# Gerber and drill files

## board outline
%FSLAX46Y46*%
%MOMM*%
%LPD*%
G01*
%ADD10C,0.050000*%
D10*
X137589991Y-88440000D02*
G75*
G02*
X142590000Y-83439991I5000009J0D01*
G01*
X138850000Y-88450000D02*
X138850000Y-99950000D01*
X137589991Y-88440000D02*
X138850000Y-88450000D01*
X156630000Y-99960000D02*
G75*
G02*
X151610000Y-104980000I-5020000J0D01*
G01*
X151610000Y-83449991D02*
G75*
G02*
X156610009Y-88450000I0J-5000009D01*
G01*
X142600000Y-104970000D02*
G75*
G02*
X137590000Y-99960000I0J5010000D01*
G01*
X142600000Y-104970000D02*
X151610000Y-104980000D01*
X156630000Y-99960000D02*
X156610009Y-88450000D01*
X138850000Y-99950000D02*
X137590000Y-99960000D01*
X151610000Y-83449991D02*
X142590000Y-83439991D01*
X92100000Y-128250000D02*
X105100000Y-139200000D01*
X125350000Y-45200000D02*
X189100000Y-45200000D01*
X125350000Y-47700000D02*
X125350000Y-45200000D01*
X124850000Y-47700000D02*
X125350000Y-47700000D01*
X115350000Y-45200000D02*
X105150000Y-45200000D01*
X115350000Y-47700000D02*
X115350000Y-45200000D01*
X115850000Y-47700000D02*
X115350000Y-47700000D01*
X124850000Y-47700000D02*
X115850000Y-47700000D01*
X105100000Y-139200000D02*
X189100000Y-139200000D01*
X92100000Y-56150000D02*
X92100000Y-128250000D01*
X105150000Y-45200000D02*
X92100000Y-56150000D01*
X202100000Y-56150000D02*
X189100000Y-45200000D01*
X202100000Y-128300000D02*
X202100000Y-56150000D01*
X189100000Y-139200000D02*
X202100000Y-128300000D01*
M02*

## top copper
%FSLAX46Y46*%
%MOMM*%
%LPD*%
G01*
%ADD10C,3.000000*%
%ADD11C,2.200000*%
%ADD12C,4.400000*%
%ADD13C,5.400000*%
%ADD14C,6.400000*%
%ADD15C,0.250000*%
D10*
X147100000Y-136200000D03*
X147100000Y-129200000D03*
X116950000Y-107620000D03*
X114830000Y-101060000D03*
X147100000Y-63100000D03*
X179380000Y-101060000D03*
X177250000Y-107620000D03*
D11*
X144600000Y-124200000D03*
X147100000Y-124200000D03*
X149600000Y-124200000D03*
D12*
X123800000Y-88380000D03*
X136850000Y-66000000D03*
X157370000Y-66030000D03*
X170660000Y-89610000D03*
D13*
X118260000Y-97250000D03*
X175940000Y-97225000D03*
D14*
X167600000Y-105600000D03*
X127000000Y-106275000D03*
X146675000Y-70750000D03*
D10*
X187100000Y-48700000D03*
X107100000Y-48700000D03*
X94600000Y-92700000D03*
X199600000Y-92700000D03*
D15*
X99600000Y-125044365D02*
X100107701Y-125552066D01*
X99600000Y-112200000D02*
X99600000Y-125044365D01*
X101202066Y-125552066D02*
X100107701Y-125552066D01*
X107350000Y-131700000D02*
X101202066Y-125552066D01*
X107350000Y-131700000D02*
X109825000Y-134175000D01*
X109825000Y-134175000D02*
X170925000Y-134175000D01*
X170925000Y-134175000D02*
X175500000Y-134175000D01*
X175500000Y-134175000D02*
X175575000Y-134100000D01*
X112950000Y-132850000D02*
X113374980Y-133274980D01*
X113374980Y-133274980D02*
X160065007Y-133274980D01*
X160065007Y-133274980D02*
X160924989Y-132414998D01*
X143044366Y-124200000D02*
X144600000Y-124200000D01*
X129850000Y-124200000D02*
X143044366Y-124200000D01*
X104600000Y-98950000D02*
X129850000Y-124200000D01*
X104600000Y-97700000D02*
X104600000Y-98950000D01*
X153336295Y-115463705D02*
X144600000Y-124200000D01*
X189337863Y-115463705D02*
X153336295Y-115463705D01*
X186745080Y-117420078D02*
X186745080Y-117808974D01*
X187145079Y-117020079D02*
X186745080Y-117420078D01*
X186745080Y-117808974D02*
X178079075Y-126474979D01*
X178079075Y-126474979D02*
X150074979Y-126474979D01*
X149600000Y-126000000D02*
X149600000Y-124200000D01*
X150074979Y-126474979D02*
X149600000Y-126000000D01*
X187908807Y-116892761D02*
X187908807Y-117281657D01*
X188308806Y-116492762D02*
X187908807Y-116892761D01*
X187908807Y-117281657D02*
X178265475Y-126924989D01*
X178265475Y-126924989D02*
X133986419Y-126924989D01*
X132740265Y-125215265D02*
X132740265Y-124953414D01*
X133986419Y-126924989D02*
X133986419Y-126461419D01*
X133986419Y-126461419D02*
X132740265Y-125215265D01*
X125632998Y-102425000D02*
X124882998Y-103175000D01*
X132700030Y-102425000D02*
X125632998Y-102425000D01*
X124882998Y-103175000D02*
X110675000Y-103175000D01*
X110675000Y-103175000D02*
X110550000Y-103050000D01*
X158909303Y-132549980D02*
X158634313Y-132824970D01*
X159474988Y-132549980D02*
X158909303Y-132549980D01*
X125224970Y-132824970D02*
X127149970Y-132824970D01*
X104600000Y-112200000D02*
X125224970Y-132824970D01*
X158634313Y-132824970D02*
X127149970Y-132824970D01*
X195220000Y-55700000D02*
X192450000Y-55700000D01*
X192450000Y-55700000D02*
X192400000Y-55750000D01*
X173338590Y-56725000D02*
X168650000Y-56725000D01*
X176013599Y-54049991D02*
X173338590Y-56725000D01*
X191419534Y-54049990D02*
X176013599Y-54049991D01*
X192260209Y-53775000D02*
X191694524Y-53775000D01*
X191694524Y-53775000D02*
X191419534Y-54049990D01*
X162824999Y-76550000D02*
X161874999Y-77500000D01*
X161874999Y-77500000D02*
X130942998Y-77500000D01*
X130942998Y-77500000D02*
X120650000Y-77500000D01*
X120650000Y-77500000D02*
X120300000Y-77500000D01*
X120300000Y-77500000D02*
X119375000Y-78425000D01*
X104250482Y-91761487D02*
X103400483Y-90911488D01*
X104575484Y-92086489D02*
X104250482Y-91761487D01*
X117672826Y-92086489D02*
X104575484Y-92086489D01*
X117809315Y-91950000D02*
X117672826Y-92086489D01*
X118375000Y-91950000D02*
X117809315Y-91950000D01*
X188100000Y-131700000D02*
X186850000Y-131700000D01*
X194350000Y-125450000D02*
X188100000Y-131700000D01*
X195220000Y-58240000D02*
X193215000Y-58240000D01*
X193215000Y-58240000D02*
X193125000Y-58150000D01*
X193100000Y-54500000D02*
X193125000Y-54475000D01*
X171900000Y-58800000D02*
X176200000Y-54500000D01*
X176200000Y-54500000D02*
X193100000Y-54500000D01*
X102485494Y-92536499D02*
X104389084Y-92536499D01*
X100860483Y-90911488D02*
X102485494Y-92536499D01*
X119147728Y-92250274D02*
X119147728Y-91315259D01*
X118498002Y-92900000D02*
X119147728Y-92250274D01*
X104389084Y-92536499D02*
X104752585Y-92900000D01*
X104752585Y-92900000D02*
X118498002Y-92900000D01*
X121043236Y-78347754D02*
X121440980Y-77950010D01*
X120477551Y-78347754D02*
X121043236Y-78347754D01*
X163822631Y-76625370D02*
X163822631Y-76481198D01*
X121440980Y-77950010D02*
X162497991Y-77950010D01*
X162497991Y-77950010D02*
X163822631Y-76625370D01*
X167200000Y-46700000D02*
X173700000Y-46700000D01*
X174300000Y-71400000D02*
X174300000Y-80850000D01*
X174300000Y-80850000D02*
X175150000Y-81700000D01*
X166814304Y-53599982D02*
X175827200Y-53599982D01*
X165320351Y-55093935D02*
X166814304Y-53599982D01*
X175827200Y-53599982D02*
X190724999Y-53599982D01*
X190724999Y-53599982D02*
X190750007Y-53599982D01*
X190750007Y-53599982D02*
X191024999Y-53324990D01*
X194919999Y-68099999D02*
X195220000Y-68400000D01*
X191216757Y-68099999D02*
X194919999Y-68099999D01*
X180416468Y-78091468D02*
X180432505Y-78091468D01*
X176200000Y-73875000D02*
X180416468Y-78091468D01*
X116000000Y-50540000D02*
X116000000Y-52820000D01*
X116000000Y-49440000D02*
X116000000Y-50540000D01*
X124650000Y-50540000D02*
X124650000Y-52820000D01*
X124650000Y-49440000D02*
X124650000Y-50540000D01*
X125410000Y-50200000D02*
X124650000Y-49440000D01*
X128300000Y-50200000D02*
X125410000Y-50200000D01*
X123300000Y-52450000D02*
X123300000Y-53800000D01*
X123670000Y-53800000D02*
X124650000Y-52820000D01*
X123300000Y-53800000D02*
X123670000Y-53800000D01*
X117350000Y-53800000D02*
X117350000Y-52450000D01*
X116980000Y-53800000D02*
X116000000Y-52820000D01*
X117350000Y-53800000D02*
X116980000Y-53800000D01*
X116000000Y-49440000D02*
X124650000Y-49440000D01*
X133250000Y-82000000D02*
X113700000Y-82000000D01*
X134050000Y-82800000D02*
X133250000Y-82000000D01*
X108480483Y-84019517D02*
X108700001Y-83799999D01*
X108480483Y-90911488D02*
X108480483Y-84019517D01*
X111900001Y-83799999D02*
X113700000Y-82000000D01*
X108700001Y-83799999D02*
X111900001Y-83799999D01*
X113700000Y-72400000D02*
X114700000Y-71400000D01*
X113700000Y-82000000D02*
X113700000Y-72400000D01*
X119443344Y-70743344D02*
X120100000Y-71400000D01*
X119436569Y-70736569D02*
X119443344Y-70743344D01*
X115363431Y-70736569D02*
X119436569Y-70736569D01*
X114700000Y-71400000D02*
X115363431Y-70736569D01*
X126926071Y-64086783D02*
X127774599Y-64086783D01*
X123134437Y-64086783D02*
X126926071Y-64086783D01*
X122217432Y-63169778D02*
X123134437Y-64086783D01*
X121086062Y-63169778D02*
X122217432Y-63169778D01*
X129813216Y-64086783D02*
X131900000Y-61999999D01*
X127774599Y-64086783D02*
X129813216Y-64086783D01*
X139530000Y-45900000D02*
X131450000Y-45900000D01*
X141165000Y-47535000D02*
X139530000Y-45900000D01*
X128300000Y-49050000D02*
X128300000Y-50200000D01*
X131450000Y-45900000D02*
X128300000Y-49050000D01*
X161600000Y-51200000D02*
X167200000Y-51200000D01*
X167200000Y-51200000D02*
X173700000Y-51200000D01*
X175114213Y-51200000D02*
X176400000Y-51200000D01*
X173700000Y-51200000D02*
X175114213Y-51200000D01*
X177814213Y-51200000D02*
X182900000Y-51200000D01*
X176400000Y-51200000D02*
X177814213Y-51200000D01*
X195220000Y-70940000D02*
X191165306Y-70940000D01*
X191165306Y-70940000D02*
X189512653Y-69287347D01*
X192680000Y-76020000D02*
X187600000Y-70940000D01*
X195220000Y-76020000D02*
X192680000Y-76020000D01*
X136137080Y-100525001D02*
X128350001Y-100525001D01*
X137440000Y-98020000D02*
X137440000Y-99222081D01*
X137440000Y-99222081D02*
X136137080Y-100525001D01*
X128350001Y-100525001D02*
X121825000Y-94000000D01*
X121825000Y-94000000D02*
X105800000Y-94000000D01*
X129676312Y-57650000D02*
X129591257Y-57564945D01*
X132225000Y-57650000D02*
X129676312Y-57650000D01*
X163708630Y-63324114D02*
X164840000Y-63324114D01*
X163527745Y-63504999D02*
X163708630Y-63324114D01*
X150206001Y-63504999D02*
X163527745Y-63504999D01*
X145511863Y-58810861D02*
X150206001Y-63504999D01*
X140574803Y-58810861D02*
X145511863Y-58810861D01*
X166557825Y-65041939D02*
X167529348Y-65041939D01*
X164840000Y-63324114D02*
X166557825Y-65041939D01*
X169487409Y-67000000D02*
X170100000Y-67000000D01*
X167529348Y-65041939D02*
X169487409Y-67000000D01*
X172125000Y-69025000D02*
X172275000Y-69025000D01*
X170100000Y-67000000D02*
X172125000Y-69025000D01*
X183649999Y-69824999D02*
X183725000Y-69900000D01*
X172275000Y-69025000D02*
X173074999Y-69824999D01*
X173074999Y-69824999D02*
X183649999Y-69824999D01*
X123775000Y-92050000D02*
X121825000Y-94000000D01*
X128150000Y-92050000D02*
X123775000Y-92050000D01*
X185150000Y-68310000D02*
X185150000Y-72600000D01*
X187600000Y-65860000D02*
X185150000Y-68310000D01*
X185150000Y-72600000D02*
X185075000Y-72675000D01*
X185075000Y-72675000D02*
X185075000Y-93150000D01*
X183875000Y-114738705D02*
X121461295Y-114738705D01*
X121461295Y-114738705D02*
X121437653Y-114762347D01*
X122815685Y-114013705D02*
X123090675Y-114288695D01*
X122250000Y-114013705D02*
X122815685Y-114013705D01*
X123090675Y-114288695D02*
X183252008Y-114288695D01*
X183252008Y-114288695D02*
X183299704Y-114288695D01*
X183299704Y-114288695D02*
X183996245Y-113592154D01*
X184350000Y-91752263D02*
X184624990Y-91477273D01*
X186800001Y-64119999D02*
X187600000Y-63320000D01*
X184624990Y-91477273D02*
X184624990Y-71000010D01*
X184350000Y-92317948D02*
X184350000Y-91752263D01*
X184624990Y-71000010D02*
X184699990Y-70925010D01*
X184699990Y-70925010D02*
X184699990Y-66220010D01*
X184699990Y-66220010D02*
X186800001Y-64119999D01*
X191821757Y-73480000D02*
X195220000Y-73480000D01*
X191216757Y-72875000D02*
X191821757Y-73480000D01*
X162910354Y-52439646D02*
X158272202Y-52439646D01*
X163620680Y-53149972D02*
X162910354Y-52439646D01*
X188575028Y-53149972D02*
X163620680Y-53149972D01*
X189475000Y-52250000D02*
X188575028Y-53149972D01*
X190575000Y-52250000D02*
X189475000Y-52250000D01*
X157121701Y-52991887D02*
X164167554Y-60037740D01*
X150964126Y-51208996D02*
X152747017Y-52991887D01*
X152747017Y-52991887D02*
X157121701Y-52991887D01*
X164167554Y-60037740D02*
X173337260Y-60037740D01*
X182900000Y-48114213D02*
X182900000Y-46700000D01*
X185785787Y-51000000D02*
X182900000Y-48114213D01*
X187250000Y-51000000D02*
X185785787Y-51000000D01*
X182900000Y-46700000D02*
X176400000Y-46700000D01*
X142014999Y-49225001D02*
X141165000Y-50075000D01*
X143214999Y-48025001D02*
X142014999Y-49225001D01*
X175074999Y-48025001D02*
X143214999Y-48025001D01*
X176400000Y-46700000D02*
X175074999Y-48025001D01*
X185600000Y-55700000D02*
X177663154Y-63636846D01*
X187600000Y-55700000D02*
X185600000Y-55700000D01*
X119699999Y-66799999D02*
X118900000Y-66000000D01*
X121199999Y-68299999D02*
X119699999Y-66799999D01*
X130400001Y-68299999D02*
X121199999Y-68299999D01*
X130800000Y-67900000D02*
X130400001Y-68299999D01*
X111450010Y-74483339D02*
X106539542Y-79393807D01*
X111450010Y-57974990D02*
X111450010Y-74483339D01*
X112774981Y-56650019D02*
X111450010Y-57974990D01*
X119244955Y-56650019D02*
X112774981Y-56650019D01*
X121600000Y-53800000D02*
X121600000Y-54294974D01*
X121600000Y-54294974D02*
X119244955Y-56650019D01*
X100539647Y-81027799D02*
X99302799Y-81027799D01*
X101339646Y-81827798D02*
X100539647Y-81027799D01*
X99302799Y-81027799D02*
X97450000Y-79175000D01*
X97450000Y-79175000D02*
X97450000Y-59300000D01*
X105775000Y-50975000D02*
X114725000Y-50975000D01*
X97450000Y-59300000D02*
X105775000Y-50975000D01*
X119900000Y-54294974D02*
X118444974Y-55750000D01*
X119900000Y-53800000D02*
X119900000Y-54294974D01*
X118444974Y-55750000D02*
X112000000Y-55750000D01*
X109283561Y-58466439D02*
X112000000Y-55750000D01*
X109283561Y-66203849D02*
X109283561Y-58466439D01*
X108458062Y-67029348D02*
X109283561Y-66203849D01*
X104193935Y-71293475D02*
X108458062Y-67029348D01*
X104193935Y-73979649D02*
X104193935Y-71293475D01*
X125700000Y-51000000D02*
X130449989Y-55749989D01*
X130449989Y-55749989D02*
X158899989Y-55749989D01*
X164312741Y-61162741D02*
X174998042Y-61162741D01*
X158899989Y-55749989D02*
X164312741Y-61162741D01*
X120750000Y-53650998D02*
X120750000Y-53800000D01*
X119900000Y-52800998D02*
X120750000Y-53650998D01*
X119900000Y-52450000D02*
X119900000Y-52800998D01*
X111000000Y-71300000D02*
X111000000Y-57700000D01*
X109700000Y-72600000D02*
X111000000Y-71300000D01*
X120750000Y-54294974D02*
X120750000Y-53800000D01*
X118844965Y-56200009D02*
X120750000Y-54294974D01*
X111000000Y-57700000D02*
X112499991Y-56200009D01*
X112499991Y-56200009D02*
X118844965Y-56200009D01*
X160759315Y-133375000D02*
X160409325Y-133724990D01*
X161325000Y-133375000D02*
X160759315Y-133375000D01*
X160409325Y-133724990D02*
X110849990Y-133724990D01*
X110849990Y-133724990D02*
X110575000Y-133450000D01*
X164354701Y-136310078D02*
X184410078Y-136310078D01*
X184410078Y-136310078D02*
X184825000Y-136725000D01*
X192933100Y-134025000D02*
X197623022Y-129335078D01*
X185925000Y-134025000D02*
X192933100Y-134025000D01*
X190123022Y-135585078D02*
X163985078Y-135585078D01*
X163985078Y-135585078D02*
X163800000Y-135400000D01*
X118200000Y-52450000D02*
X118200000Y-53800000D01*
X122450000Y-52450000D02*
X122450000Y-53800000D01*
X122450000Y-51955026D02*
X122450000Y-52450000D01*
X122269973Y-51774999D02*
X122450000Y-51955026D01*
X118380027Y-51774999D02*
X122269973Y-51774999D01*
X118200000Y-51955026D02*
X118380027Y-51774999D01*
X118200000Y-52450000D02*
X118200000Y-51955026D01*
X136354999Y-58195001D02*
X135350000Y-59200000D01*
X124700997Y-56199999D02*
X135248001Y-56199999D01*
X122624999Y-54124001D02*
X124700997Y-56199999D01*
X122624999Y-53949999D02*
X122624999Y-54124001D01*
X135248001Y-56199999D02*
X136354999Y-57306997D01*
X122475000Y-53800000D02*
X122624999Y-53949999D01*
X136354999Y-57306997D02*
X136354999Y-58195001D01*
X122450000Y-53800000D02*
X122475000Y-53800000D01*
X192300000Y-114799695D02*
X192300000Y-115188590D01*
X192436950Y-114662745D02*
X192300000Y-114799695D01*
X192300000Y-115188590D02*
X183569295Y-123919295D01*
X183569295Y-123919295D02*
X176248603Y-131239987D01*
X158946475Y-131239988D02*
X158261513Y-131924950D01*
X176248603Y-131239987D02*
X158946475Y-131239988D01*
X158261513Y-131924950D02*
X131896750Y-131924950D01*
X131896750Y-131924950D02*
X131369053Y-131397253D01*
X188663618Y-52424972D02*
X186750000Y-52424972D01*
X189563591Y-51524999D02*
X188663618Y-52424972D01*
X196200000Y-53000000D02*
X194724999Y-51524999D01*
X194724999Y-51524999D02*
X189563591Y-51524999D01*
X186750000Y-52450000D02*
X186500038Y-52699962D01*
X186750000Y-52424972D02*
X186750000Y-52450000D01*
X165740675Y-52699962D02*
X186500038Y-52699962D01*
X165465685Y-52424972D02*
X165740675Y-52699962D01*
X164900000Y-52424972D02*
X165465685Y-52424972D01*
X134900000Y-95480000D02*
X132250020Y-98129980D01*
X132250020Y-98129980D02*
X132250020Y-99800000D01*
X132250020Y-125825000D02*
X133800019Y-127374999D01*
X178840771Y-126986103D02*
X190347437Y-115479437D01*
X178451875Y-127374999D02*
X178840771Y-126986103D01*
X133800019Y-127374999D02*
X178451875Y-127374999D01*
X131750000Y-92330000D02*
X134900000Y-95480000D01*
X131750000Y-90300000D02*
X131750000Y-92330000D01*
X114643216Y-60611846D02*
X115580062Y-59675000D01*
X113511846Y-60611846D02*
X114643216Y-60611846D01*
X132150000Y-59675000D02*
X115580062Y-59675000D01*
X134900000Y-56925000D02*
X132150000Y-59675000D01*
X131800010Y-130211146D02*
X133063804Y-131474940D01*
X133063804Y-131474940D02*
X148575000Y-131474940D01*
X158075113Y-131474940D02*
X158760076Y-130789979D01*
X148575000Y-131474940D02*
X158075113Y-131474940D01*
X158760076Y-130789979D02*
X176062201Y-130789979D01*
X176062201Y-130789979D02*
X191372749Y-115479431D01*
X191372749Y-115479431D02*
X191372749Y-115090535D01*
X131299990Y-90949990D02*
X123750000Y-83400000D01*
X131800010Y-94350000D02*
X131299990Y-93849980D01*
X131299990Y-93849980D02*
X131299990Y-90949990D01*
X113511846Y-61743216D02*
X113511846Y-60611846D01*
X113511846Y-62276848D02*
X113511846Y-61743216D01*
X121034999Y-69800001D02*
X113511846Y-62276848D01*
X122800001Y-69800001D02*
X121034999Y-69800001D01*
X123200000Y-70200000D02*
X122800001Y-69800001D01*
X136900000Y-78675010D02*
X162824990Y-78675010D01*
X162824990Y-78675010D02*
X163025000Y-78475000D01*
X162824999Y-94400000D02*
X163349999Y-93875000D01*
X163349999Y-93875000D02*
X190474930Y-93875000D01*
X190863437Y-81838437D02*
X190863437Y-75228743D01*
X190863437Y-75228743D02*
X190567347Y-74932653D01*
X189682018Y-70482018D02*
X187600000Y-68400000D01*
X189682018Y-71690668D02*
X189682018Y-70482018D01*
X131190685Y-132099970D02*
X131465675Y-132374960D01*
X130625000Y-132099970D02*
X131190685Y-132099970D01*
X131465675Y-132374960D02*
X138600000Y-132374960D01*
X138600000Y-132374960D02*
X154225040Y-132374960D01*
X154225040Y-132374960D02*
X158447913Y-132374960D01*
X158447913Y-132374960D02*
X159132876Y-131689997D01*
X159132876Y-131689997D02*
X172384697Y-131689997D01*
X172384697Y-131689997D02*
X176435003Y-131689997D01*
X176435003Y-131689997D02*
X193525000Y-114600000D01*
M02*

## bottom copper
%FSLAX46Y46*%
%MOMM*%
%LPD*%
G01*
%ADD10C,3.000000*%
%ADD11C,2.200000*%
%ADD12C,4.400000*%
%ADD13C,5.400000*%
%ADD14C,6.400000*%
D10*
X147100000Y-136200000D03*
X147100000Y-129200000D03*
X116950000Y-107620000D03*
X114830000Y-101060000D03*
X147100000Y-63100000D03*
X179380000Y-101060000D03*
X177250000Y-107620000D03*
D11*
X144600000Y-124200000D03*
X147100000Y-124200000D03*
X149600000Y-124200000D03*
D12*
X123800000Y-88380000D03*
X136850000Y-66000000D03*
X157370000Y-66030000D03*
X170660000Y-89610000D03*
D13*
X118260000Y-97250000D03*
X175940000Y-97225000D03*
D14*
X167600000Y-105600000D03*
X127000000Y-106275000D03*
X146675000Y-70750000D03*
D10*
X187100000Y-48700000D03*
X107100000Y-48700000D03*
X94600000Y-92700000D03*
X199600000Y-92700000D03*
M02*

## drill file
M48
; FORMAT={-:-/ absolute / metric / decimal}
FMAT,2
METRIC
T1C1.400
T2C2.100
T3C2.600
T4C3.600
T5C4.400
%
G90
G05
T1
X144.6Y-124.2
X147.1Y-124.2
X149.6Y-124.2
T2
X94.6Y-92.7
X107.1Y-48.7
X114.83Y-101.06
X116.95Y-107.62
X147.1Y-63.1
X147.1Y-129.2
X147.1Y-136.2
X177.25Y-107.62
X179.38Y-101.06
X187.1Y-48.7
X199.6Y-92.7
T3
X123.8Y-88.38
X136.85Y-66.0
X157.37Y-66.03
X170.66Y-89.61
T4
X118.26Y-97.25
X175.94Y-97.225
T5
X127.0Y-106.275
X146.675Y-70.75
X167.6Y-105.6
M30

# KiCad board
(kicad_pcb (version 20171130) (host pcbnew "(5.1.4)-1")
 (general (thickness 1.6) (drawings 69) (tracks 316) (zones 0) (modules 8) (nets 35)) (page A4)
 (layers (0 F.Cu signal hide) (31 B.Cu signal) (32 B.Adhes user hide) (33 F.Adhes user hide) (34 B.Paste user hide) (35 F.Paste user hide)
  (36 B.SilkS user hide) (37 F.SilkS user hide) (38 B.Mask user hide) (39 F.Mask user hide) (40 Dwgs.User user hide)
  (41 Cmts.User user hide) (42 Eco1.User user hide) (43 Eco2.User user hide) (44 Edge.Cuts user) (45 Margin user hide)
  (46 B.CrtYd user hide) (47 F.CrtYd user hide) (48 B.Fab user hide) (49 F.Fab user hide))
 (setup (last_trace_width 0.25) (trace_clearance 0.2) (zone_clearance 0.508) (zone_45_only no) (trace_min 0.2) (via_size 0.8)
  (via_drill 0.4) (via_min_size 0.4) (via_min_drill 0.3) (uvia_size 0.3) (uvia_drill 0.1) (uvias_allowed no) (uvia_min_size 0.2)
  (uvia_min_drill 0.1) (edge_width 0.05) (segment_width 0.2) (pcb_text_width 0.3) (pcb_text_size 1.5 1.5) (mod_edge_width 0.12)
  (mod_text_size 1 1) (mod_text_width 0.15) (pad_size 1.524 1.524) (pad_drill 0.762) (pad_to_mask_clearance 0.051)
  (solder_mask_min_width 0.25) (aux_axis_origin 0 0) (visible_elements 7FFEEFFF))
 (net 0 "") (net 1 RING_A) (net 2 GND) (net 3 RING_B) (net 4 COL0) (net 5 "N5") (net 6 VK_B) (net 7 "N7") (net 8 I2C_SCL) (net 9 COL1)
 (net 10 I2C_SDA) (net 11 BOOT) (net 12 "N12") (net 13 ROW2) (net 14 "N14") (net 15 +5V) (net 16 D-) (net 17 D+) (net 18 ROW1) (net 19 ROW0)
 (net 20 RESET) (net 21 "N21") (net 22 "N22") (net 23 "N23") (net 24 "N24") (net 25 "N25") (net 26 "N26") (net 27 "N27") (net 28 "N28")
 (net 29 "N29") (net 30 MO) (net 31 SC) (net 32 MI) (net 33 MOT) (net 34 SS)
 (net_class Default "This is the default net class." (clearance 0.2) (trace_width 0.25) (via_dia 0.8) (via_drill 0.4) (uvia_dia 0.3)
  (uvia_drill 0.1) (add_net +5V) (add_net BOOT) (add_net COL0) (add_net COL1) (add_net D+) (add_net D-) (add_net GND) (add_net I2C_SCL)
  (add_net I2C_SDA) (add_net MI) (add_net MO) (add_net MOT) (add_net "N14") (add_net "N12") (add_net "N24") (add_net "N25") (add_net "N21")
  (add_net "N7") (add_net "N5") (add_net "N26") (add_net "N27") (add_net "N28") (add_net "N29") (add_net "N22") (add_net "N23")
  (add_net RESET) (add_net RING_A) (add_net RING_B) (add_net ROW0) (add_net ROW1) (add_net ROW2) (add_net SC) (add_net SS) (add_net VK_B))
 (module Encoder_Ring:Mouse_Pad (layer F.Cu) (at 147.1 94.2)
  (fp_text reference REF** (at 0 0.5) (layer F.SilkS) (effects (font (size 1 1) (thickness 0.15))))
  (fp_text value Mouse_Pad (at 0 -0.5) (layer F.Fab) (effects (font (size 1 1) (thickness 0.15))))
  (pad "" thru_hole circle (at 0 42) (size 3 3) (drill 2.1) (layers *.Cu *.Mask))
  (pad "" thru_hole circle (at 0 35) (size 3 3) (drill 2.1) (layers *.Cu *.Mask))
  (pad "" thru_hole circle (at -30.15 13.42) (size 3 3) (drill 2.1) (layers *.Cu *.Mask))
  (pad "" thru_hole circle (at -32.27 6.86) (size 3 3) (drill 2.1) (layers *.Cu *.Mask))
  (pad "" thru_hole circle (at 0 -31.1) (size 3 3) (drill 2.1) (layers *.Cu *.Mask))
  (pad "" thru_hole circle (at 32.28 6.86) (size 3 3) (drill 2.1) (layers *.Cu *.Mask))
  (pad "" thru_hole circle (at 30.15 13.42) (size 3 3) (drill 2.1) (layers *.Cu *.Mask)))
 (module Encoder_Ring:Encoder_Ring (layer F.Cu) (at 147.1 94.2)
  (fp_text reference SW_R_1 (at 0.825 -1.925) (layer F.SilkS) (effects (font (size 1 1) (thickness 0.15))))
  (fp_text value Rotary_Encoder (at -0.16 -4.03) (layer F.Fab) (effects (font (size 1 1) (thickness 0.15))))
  (pad A thru_hole circle (at -2.5 30) (size 2.2 2.2) (drill 1.4) (layers *.Cu *.Mask) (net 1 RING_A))
  (pad C thru_hole circle (at 0 30) (size 2.2 2.2) (drill 1.4) (layers *.Cu *.Mask) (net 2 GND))
  (pad B thru_hole circle (at 2.5 30) (size 2.2 2.2) (drill 1.4) (layers *.Cu *.Mask) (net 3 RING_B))
  (pad "" thru_hole circle (at -23.3 -5.82) (size 4.4 4.4) (drill 2.6) (layers *.Cu *.Mask))
  (pad "" thru_hole circle (at -10.25 -28.2) (size 4.4 4.4) (drill 2.6) (layers *.Cu *.Mask))
  (pad "" thru_hole circle (at 10.27 -28.17) (size 4.4 4.4) (drill 2.6) (layers *.Cu *.Mask))
  (pad "" thru_hole circle (at 23.56 -4.59) (size 4.4 4.4) (drill 2.6) (layers *.Cu *.Mask))
  (pad "" thru_hole circle (at -28.84 3.05) (size 5.4 5.4) (drill 3.6) (layers *.Cu *.Mask))
  (pad "" thru_hole circle (at 28.84 3.025) (size 5.4 5.4) (drill 3.6) (layers *.Cu *.Mask))
  (pad "" thru_hole circle (at 20.5 11.4) (size 6.4 6.4) (drill 4.4) (layers *.Cu *.Mask))
  (pad "" thru_hole circle (at -20.1 12.075) (size 6.4 6.4) (drill 4.4) (layers *.Cu *.Mask))
  (pad "" thru_hole circle (at -0.425 -23.45) (size 6.4 6.4) (drill 4.4) (layers *.Cu *.Mask)))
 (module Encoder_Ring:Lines (layer F.Cu) (at 147 92.1)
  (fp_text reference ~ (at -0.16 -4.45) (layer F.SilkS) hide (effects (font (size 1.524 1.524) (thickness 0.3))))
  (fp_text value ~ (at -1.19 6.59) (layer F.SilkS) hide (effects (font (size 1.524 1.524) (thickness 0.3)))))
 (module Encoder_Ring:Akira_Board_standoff (layer F.Cu) (at 187.1 48.7)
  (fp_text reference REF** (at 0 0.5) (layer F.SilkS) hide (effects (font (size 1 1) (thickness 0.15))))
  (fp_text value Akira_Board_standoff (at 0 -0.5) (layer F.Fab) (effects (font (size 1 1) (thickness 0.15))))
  (pad "" thru_hole circle (at 0 0) (size 3 3) (drill 2.1) (layers *.Cu *.Mask)))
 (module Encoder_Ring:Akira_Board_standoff (layer F.Cu) (at 107.1 48.7)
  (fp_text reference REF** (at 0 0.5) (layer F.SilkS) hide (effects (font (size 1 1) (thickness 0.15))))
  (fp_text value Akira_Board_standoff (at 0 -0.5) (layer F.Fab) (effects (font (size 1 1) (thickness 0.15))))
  (pad "" thru_hole circle (at 0 0) (size 3 3) (drill 2.1) (layers *.Cu *.Mask)))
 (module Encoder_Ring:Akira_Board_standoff (layer F.Cu) (at 94.6 92.7)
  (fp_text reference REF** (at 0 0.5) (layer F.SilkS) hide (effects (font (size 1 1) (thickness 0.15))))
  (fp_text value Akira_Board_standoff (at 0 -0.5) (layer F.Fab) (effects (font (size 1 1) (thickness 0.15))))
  (pad "" thru_hole circle (at 0 0) (size 3 3) (drill 2.1) (layers *.Cu *.Mask)))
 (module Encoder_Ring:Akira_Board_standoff (layer F.Cu) (at 199.6 92.7)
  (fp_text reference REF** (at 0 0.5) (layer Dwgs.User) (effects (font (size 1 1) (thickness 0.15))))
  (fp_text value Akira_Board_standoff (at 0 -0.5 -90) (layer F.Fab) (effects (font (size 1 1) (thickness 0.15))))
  (pad "" thru_hole circle (at 0 0) (size 3 3) (drill 2.1) (layers *.Cu *.Mask)))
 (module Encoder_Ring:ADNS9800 (layer F.Cu) (at 147.1 94.2)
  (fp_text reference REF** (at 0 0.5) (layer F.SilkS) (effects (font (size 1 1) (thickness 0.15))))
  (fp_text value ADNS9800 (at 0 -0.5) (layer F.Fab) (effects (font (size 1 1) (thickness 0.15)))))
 (gr_arc (start 142.59 88.44) (end 142.59 83.439991) (angle -90) (layer Edge.Cuts) (width 0.05))
 (gr_line (start 138.85 88.45) (end 138.85 99.95) (layer Edge.Cuts) (width 0.05))
 (gr_line (start 137.589991 88.44) (end 138.85 88.45) (layer Edge.Cuts) (width 0.05))
 (gr_arc (start 151.61 99.96) (end 151.61 104.98) (angle -90) (layer Edge.Cuts) (width 0.05))
 (gr_arc (start 151.61 88.45) (end 156.610009 88.45) (angle -90) (layer Edge.Cuts) (width 0.05))
 (gr_arc (start 142.6 99.96) (end 137.59 99.96) (angle -90) (layer Edge.Cuts) (width 0.05))
 (gr_line (start 142.6 104.97) (end 151.61 104.98) (layer Edge.Cuts) (width 0.05))
 (gr_line (start 156.63 99.96) (end 156.610009 88.45) (layer Edge.Cuts) (width 0.05))
 (gr_line (start 138.85 99.95) (end 137.59 99.96) (layer Edge.Cuts) (width 0.05))
 (gr_line (start 151.61 83.449991) (end 142.59 83.439991) (layer Edge.Cuts) (width 0.05))
 (gr_line (start 92.1 128.25) (end 105.1 139.2) (layer Edge.Cuts) (width 0.05))
 (gr_line (start 125.35 45.2) (end 189.1 45.2) (layer Edge.Cuts) (width 0.05))
 (gr_line (start 125.35 47.7) (end 125.35 45.2) (layer Edge.Cuts) (width 0.05))
 (gr_line (start 124.85 47.7) (end 125.35 47.7) (layer Edge.Cuts) (width 0.05))
 (gr_line (start 115.35 45.2) (end 105.15 45.2) (layer Edge.Cuts) (width 0.05))
 (gr_line (start 115.35 47.7) (end 115.35 45.2) (layer Edge.Cuts) (width 0.05))
 (gr_line (start 115.85 47.7) (end 115.35 47.7) (layer Edge.Cuts) (width 0.05))
 (gr_line (start 124.85 47.7) (end 115.85 47.7) (layer Edge.Cuts) (width 0.05))
 (gr_line (start 105.1 139.2) (end 189.1 139.2) (layer Edge.Cuts) (width 0.05))
 (gr_line (start 92.1 56.15) (end 92.1 128.25) (layer Edge.Cuts) (width 0.05))
 (gr_line (start 105.15 45.2) (end 92.1 56.15) (layer Edge.Cuts) (width 0.05))
 (gr_line (start 202.1 56.15) (end 189.1 45.2) (layer Edge.Cuts) (width 0.05))
 (gr_line (start 202.1 128.3) (end 202.1 56.15) (layer Edge.Cuts) (width 0.05))
 (gr_line (start 189.1 139.2) (end 202.1 128.3) (layer Edge.Cuts) (width 0.05))
 (segment (start 99.6 125.044365) (end 100.107701 125.552066) (width 0.25) (layer F.Cu) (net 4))
 (segment (start 99.6 112.2) (end 99.6 125.044365) (width 0.25) (layer F.Cu) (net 4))
 (segment (start 101.202066 125.552066) (end 100.107701 125.552066) (width 0.25) (layer F.Cu) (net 4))
 (segment (start 107.35 131.7) (end 101.202066 125.552066) (width 0.25) (layer F.Cu) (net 4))
 (segment (start 107.35 131.7) (end 109.825 134.175) (width 0.25) (layer F.Cu) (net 4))
 (segment (start 109.825 134.175) (end 170.925 134.175) (width 0.25) (layer F.Cu) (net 4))
 (segment (start 170.925 134.175) (end 175.5 134.175) (width 0.25) (layer F.Cu) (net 4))
 (segment (start 175.5 134.175) (end 175.575 134.1) (width 0.25) (layer F.Cu) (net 4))
 (segment (start 112.95 132.85) (end 113.37498 133.27498) (width 0.25) (layer F.Cu) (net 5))
 (segment (start 113.37498 133.27498) (end 160.065007 133.27498) (width 0.25) (layer F.Cu) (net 5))
 (segment (start 160.065007 133.27498) (end 160.924989 132.414998) (width 0.25) (layer F.Cu) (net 5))
 (segment (start 143.044366 124.2) (end 144.6 124.2) (width 0.25) (layer F.Cu) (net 1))
 (segment (start 129.85 124.2) (end 143.044366 124.2) (width 0.25) (layer F.Cu) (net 1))
 (segment (start 104.6 98.95) (end 129.85 124.2) (width 0.25) (layer F.Cu) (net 1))
 (segment (start 104.6 97.7) (end 104.6 98.95) (width 0.25) (layer F.Cu) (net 1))
 (segment (start 153.336295 115.463705) (end 144.6 124.2) (width 0.25) (layer F.Cu) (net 1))
 (segment (start 189.337863 115.463705) (end 153.336295 115.463705) (width 0.25) (layer F.Cu) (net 1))
 (segment (start 186.74508 117.420078) (end 186.74508 117.808974) (width 0.25) (layer F.Cu) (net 3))
 (segment (start 187.145079 117.020079) (end 186.74508 117.420078) (width 0.25) (layer F.Cu) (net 3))
 (segment (start 186.74508 117.808974) (end 178.079075 126.474979) (width 0.25) (layer F.Cu) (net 3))
 (segment (start 178.079075 126.474979) (end 150.074979 126.474979) (width 0.25) (layer F.Cu) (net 3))
 (segment (start 149.6 126) (end 149.6 124.2) (width 0.25) (layer F.Cu) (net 3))
 (segment (start 150.074979 126.474979) (end 149.6 126) (width 0.25) (layer F.Cu) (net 3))
 (segment (start 187.908807 116.892761) (end 187.908807 117.281657) (width 0.25) (layer F.Cu) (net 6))
 (segment (start 188.308806 116.492762) (end 187.908807 116.892761) (width 0.25) (layer F.Cu) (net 6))
 (segment (start 187.908807 117.281657) (end 178.265475 126.924989) (width 0.25) (layer F.Cu) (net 6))
 (segment (start 178.265475 126.924989) (end 133.986419 126.924989) (width 0.25) (layer F.Cu) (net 6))
 (segment (start 132.740265 125.215265) (end 132.740265 124.953414) (width 0.25) (layer F.Cu) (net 6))
 (segment (start 133.986419 126.924989) (end 133.986419 126.461419) (width 0.25) (layer F.Cu) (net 6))
 (segment (start 133.986419 126.461419) (end 132.740265 125.215265) (width 0.25) (layer F.Cu) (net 6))
 (segment (start 125.632998 102.425) (end 124.882998 103.175) (width 0.25) (layer F.Cu) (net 6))
 (segment (start 132.70003 102.425) (end 125.632998 102.425) (width 0.25) (layer F.Cu) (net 6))
 (segment (start 124.882998 103.175) (end 110.675 103.175) (width 0.25) (layer F.Cu) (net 6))
 (segment (start 110.675 103.175) (end 110.55 103.05) (width 0.25) (layer F.Cu) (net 6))
 (segment (start 158.909303 132.54998) (end 158.634313 132.82497) (width 0.25) (layer F.Cu) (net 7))
 (segment (start 159.474988 132.54998) (end 158.909303 132.54998) (width 0.25) (layer F.Cu) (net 7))
 (segment (start 125.22497 132.82497) (end 127.14997 132.82497) (width 0.25) (layer F.Cu) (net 7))
 (segment (start 104.6 112.2) (end 125.22497 132.82497) (width 0.25) (layer F.Cu) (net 7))
 (segment (start 158.634313 132.82497) (end 127.14997 132.82497) (width 0.25) (layer F.Cu) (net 7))
 (segment (start 195.22 55.7) (end 192.45 55.7) (width 0.25) (layer F.Cu) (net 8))
 (segment (start 192.45 55.7) (end 192.4 55.75) (width 0.25) (layer F.Cu) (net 8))
 (segment (start 173.33859 56.725) (end 168.65 56.725) (width 0.25) (layer F.Cu) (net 8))
 (segment (start 176.013599 54.049991) (end 173.33859 56.725) (width 0.25) (layer F.Cu) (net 8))
 (segment (start 191.419534 54.04999) (end 176.013599 54.049991) (width 0.25) (layer F.Cu) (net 8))
 (segment (start 192.260209 53.775) (end 191.694524 53.775) (width 0.25) (layer F.Cu) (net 8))
 (segment (start 191.694524 53.775) (end 191.419534 54.04999) (width 0.25) (layer F.Cu) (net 8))
 (segment (start 162.824999 76.55) (end 161.874999 77.5) (width 0.25) (layer F.Cu) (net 8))
 (segment (start 161.874999 77.5) (end 130.942998 77.5) (width 0.25) (layer F.Cu) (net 8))
 (segment (start 130.942998 77.5) (end 120.65 77.5) (width 0.25) (layer F.Cu) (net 8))
 (segment (start 120.65 77.5) (end 120.3 77.5) (width 0.25) (layer F.Cu) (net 8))
 (segment (start 120.3 77.5) (end 119.375 78.425) (width 0.25) (layer F.Cu) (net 8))
 (segment (start 104.250482 91.761487) (end 103.400483 90.911488) (width 0.25) (layer F.Cu) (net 8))
 (segment (start 104.575484 92.086489) (end 104.250482 91.761487) (width 0.25) (layer F.Cu) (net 8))
 (segment (start 117.672826 92.086489) (end 104.575484 92.086489) (width 0.25) (layer F.Cu) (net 8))
 (segment (start 117.809315 91.95) (end 117.672826 92.086489) (width 0.25) (layer F.Cu) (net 8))
 (segment (start 118.375 91.95) (end 117.809315 91.95) (width 0.25) (layer F.Cu) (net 8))
 (segment (start 188.1 131.7) (end 186.85 131.7) (width 0.25) (layer F.Cu) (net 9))
 (segment (start 194.35 125.45) (end 188.1 131.7) (width 0.25) (layer F.Cu) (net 9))
 (segment (start 195.22 58.24) (end 193.215 58.24) (width 0.25) (layer F.Cu) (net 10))
 (segment (start 193.215 58.24) (end 193.125 58.15) (width 0.25) (layer F.Cu) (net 10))
 (segment (start 193.1 54.5) (end 193.125 54.475) (width 0.25) (layer F.Cu) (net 10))
 (segment (start 171.9 58.8) (end 176.2 54.5) (width 0.25) (layer F.Cu) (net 10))
 (segment (start 176.2 54.5) (end 193.1 54.5) (width 0.25) (layer F.Cu) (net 10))
 (segment (start 102.485494 92.536499) (end 104.389084 92.536499) (width 0.25) (layer F.Cu) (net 10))
 (segment (start 100.860483 90.911488) (end 102.485494 92.536499) (width 0.25) (layer F.Cu) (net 10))
 (segment (start 119.147728 92.250274) (end 119.147728 91.315259) (width 0.25) (layer F.Cu) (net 10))
 (segment (start 118.498002 92.9) (end 119.147728 92.250274) (width 0.25) (layer F.Cu) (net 10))
 (segment (start 104.389084 92.536499) (end 104.752585 92.9) (width 0.25) (layer F.Cu) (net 10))
 (segment (start 104.752585 92.9) (end 118.498002 92.9) (width 0.25) (layer F.Cu) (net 10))
 (segment (start 121.043236 78.347754) (end 121.44098 77.95001) (width 0.25) (layer F.Cu) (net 10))
 (segment (start 120.477551 78.347754) (end 121.043236 78.347754) (width 0.25) (layer F.Cu) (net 10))
 (segment (start 163.822631 76.62537) (end 163.822631 76.481198) (width 0.25) (layer F.Cu) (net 10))
 (segment (start 121.44098 77.95001) (end 162.497991 77.95001) (width 0.25) (layer F.Cu) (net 10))
 (segment (start 162.497991 77.95001) (end 163.822631 76.62537) (width 0.25) (layer F.Cu) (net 10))
 (segment (start 167.2 46.7) (end 173.7 46.7) (width 0.25) (layer F.Cu) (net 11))
 (segment (start 174.3 71.4) (end 174.3 80.85) (width 0.25) (layer F.Cu) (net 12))
 (segment (start 174.3 80.85) (end 175.15 81.7) (width 0.25) (layer F.Cu) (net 12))
 (segment (start 166.814304 53.599982) (end 175.8272 53.599982) (width 0.25) (layer F.Cu) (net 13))
 (segment (start 165.320351 55.093935) (end 166.814304 53.599982) (width 0.25) (layer F.Cu) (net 13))
 (segment (start 175.8272 53.599982) (end 190.724999 53.599982) (width 0.25) (layer F.Cu) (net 13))
 (segment (start 190.724999 53.599982) (end 190.750007 53.599982) (width 0.25) (layer F.Cu) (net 13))
 (segment (start 190.750007 53.599982) (end 191.024999 53.32499) (width 0.25) (layer F.Cu) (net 13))
 (segment (start 194.919999 68.099999) (end 195.22 68.4) (width 0.25) (layer F.Cu) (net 13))
 (segment (start 191.216757 68.099999) (end 194.919999 68.099999) (width 0.25) (layer F.Cu) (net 13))
 (segment (start 180.416468 78.091468) (end 180.432505 78.091468) (width 0.25) (layer F.Cu) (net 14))
 (segment (start 176.2 73.875) (end 180.416468 78.091468) (width 0.25) (layer F.Cu) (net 14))
 (segment (start 116 50.54) (end 116 52.82) (width 0.25) (layer F.Cu) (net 2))
 (segment (start 116 49.44) (end 116 50.54) (width 0.25) (layer F.Cu) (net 2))
 (segment (start 124.65 50.54) (end 124.65 52.82) (width 0.25) (layer F.Cu) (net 2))
 (segment (start 124.65 49.44) (end 124.65 50.54) (width 0.25) (layer F.Cu) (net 2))
 (segment (start 125.41 50.2) (end 124.65 49.44) (width 0.25) (layer F.Cu) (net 2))
 (segment (start 128.3 50.2) (end 125.41 50.2) (width 0.25) (layer F.Cu) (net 2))
 (segment (start 123.3 52.45) (end 123.3 53.8) (width 0.25) (layer F.Cu) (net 2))
 (segment (start 123.67 53.8) (end 124.65 52.82) (width 0.25) (layer F.Cu) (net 2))
 (segment (start 123.3 53.8) (end 123.67 53.8) (width 0.25) (layer F.Cu) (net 2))
 (segment (start 117.35 53.8) (end 117.35 52.45) (width 0.25) (layer F.Cu) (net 2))
 (segment (start 116.98 53.8) (end 116 52.82) (width 0.25) (layer F.Cu) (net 2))
 (segment (start 117.35 53.8) (end 116.98 53.8) (width 0.25) (layer F.Cu) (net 2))
 (segment (start 116 49.44) (end 124.65 49.44) (width 0.25) (layer F.Cu) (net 2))
 (segment (start 133.25 82) (end 113.7 82) (width 0.25) (layer F.Cu) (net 2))
 (segment (start 134.05 82.8) (end 133.25 82) (width 0.25) (layer F.Cu) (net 2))
 (segment (start 108.480483 84.019517) (end 108.700001 83.799999) (width 0.25) (layer F.Cu) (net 2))
 (segment (start 108.480483 90.911488) (end 108.480483 84.019517) (width 0.25) (layer F.Cu) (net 2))
 (segment (start 111.900001 83.799999) (end 113.7 82) (width 0.25) (layer F.Cu) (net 2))
 (segment (start 108.700001 83.799999) (end 111.900001 83.799999) (width 0.25) (layer F.Cu) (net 2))
 (segment (start 113.7 72.4) (end 114.7 71.4) (width 0.25) (layer F.Cu) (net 2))
 (segment (start 113.7 82) (end 113.7 72.4) (width 0.25) (layer F.Cu) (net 2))
 (segment (start 119.443344 70.743344) (end 120.1 71.4) (width 0.25) (layer F.Cu) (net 2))
 (segment (start 119.436569 70.736569) (end 119.443344 70.743344) (width 0.25) (layer F.Cu) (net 2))
 (segment (start 115.363431 70.736569) (end 119.436569 70.736569) (width 0.25) (layer F.Cu) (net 2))
 (segment (start 114.7 71.4) (end 115.363431 70.736569) (width 0.25) (layer F.Cu) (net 2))
 (segment (start 126.926071 64.086783) (end 127.774599 64.086783) (width 0.25) (layer F.Cu) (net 2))
 (segment (start 123.134437 64.086783) (end 126.926071 64.086783) (width 0.25) (layer F.Cu) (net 2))
 (segment (start 122.217432 63.169778) (end 123.134437 64.086783) (width 0.25) (layer F.Cu) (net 2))
 (segment (start 121.086062 63.169778) (end 122.217432 63.169778) (width 0.25) (layer F.Cu) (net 2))
 (segment (start 129.813216 64.086783) (end 131.9 61.999999) (width 0.25) (layer F.Cu) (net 2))
 (segment (start 127.774599 64.086783) (end 129.813216 64.086783) (width 0.25) (layer F.Cu) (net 2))
 (segment (start 139.53 45.9) (end 131.45 45.9) (width 0.25) (layer F.Cu) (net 2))
 (segment (start 141.165 47.535) (end 139.53 45.9) (width 0.25) (layer F.Cu) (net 2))
 (segment (start 128.3 49.05) (end 128.3 50.2) (width 0.25) (layer F.Cu) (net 2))
 (segment (start 131.45 45.9) (end 128.3 49.05) (width 0.25) (layer F.Cu) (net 2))
 (segment (start 161.6 51.2) (end 167.2 51.2) (width 0.25) (layer F.Cu) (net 2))
 (segment (start 167.2 51.2) (end 173.7 51.2) (width 0.25) (layer F.Cu) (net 2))
 (segment (start 175.114213 51.2) (end 176.4 51.2) (width 0.25) (layer F.Cu) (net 2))
 (segment (start 173.7 51.2) (end 175.114213 51.2) (width 0.25) (layer F.Cu) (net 2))
 (segment (start 177.814213 51.2) (end 182.9 51.2) (width 0.25) (layer F.Cu) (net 2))
 (segment (start 176.4 51.2) (end 177.814213 51.2) (width 0.25) (layer F.Cu) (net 2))
 (segment (start 195.22 70.94) (end 191.165306 70.94) (width 0.25) (layer F.Cu) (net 2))
 (segment (start 191.165306 70.94) (end 189.512653 69.287347) (width 0.25) (layer F.Cu) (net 2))
 (segment (start 192.68 76.02) (end 187.6 70.94) (width 0.25) (layer F.Cu) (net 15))
 (segment (start 195.22 76.02) (end 192.68 76.02) (width 0.25) (layer F.Cu) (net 15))
 (segment (start 136.13708 100.525001) (end 128.350001 100.525001) (width 0.25) (layer F.Cu) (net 15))
 (segment (start 137.44 98.02) (end 137.44 99.222081) (width 0.25) (layer F.Cu) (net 15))
 (segment (start 137.44 99.222081) (end 136.13708 100.525001) (width 0.25) (layer F.Cu) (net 15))
 (segment (start 128.350001 100.525001) (end 121.825 94) (width 0.25) (layer F.Cu) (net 15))
 (segment (start 121.825 94) (end 105.8 94) (width 0.25) (layer F.Cu) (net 15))
 (segment (start 129.676312 57.65) (end 129.591257 57.564945) (width 0.25) (layer F.Cu) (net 15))
 (segment (start 132.225 57.65) (end 129.676312 57.65) (width 0.25) (layer F.Cu) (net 15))
 (segment (start 163.70863 63.324114) (end 164.84 63.324114) (width 0.25) (layer F.Cu) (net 15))
 (segment (start 163.527745 63.504999) (end 163.70863 63.324114) (width 0.25) (layer F.Cu) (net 15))
 (segment (start 150.206001 63.504999) (end 163.527745 63.504999) (width 0.25) (layer F.Cu) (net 15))
 (segment (start 145.511863 58.810861) (end 150.206001 63.504999) (width 0.25) (layer F.Cu) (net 15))
 (segment (start 140.574803 58.810861) (end 145.511863 58.810861) (width 0.25) (layer F.Cu) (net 15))
 (segment (start 166.557825 65.041939) (end 167.529348 65.041939) (width 0.25) (layer F.Cu) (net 15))
 (segment (start 164.84 63.324114) (end 166.557825 65.041939) (width 0.25) (layer F.Cu) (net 15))
 (segment (start 169.487409 67) (end 170.1 67) (width 0.25) (layer F.Cu) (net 15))
 (segment (start 167.529348 65.041939) (end 169.487409 67) (width 0.25) (layer F.Cu) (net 15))
 (segment (start 172.125 69.025) (end 172.275 69.025) (width 0.25) (layer F.Cu) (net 15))
 (segment (start 170.1 67) (end 172.125 69.025) (width 0.25) (layer F.Cu) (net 15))
 (segment (start 183.649999 69.824999) (end 183.725 69.9) (width 0.25) (layer F.Cu) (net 15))
 (segment (start 172.275 69.025) (end 173.074999 69.824999) (width 0.25) (layer F.Cu) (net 15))
 (segment (start 173.074999 69.824999) (end 183.649999 69.824999) (width 0.25) (layer F.Cu) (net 15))
 (segment (start 123.775 92.05) (end 121.825 94) (width 0.25) (layer F.Cu) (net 15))
 (segment (start 128.15 92.05) (end 123.775 92.05) (width 0.25) (layer F.Cu) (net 15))
 (segment (start 185.15 68.31) (end 185.15 72.6) (width 0.25) (layer F.Cu) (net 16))
 (segment (start 187.6 65.86) (end 185.15 68.31) (width 0.25) (layer F.Cu) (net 16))
 (segment (start 185.15 72.6) (end 185.075 72.675) (width 0.25) (layer F.Cu) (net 16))
 (segment (start 185.075 72.675) (end 185.075 93.15) (width 0.25) (layer F.Cu) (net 16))
 (segment (start 183.875 114.738705) (end 121.461295 114.738705) (width 0.25) (layer F.Cu) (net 16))
 (segment (start 121.461295 114.738705) (end 121.437653 114.762347) (width 0.25) (layer F.Cu) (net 16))
 (segment (start 122.815685 114.013705) (end 123.090675 114.288695) (width 0.25) (layer F.Cu) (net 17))
 (segment (start 122.25 114.013705) (end 122.815685 114.013705) (width 0.25) (layer F.Cu) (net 17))
 (segment (start 123.090675 114.288695) (end 183.252008 114.288695) (width 0.25) (layer F.Cu) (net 17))
 (segment (start 183.252008 114.288695) (end 183.299704 114.288695) (width 0.25) (layer F.Cu) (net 17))
 (segment (start 183.299704 114.288695) (end 183.996245 113.592154) (width 0.25) (layer F.Cu) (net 17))
 (segment (start 184.35 91.752263) (end 184.62499 91.477273) (width 0.25) (layer F.Cu) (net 17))
 (segment (start 186.800001 64.119999) (end 187.6 63.32) (width 0.25) (layer F.Cu) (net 17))
 (segment (start 184.62499 91.477273) (end 184.62499 71.00001) (width 0.25) (layer F.Cu) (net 17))
 (segment (start 184.35 92.317948) (end 184.35 91.752263) (width 0.25) (layer F.Cu) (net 17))
 (segment (start 184.62499 71.00001) (end 184.69999 70.92501) (width 0.25) (layer F.Cu) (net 17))
 (segment (start 184.69999 70.92501) (end 184.69999 66.22001) (width 0.25) (layer F.Cu) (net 17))
 (segment (start 184.69999 66.22001) (end 186.800001 64.119999) (width 0.25) (layer F.Cu) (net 17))
 (segment (start 191.821757 73.48) (end 195.22 73.48) (width 0.25) (layer F.Cu) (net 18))
 (segment (start 191.216757 72.875) (end 191.821757 73.48) (width 0.25) (layer F.Cu) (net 18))
 (segment (start 162.910354 52.439646) (end 158.272202 52.439646) (width 0.25) (layer F.Cu) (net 18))
 (segment (start 163.62068 53.149972) (end 162.910354 52.439646) (width 0.25) (layer F.Cu) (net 18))
 (segment (start 188.575028 53.149972) (end 163.62068 53.149972) (width 0.25) (layer F.Cu) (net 18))
 (segment (start 189.475 52.25) (end 188.575028 53.149972) (width 0.25) (layer F.Cu) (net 18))
 (segment (start 190.575 52.25) (end 189.475 52.25) (width 0.25) (layer F.Cu) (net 18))
 (segment (start 157.121701 52.991887) (end 164.167554 60.03774) (width 0.25) (layer F.Cu) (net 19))
 (segment (start 150.964126 51.208996) (end 152.747017 52.991887) (width 0.25) (layer F.Cu) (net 19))
 (segment (start 152.747017 52.991887) (end 157.121701 52.991887) (width 0.25) (layer F.Cu) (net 19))
 (segment (start 164.167554 60.03774) (end 173.33726 60.03774) (width 0.25) (layer F.Cu) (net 19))
 (segment (start 182.9 48.114213) (end 182.9 46.7) (width 0.25) (layer F.Cu) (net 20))
 (segment (start 185.785787 51) (end 182.9 48.114213) (width 0.25) (layer F.Cu) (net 20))
 (segment (start 187.25 51) (end 185.785787 51) (width 0.25) (layer F.Cu) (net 20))
 (segment (start 182.9 46.7) (end 176.4 46.7) (width 0.25) (layer F.Cu) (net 20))
 (segment (start 142.014999 49.225001) (end 141.165 50.075) (width 0.25) (layer F.Cu) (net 20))
 (segment (start 143.214999 48.025001) (end 142.014999 49.225001) (width 0.25) (layer F.Cu) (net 20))
 (segment (start 175.074999 48.025001) (end 143.214999 48.025001) (width 0.25) (layer F.Cu) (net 20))
 (segment (start 176.4 46.7) (end 175.074999 48.025001) (width 0.25) (layer F.Cu) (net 20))
 (segment (start 185.6 55.7) (end 177.663154 63.636846) (width 0.25) (layer F.Cu) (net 20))
 (segment (start 187.6 55.7) (end 185.6 55.7) (width 0.25) (layer F.Cu) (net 20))
 (segment (start 119.699999 66.799999) (end 118.9 66) (width 0.25) (layer F.Cu) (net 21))
 (segment (start 121.199999 68.299999) (end 119.699999 66.799999) (width 0.25) (layer F.Cu) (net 21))
 (segment (start 130.400001 68.299999) (end 121.199999 68.299999) (width 0.25) (layer F.Cu) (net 21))
 (segment (start 130.8 67.9) (end 130.400001 68.299999) (width 0.25) (layer F.Cu) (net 21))
 (segment (start 111.45001 74.483339) (end 106.539542 79.393807) (width 0.25) (layer F.Cu) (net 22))
 (segment (start 111.45001 57.97499) (end 111.45001 74.483339) (width 0.25) (layer F.Cu) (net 22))
 (segment (start 112.774981 56.650019) (end 111.45001 57.97499) (width 0.25) (layer F.Cu) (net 22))
 (segment (start 119.244955 56.650019) (end 112.774981 56.650019) (width 0.25) (layer F.Cu) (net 22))
 (segment (start 121.6 53.8) (end 121.6 54.294974) (width 0.25) (layer F.Cu) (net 22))
 (segment (start 121.6 54.294974) (end 119.244955 56.650019) (width 0.25) (layer F.Cu) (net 22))
 (segment (start 100.539647 81.027799) (end 99.302799 81.027799) (width 0.25) (layer F.Cu) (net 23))
 (segment (start 101.339646 81.827798) (end 100.539647 81.027799) (width 0.25) (layer F.Cu) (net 23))
 (segment (start 99.302799 81.027799) (end 97.45 79.175) (width 0.25) (layer F.Cu) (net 23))
 (segment (start 97.45 79.175) (end 97.45 59.3) (width 0.25) (layer F.Cu) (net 23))
 (segment (start 105.775 50.975) (end 114.725 50.975) (width 0.25) (layer F.Cu) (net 23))
 (segment (start 97.45 59.3) (end 105.775 50.975) (width 0.25) (layer F.Cu) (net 23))
 (segment (start 119.9 54.294974) (end 118.444974 55.75) (width 0.25) (layer F.Cu) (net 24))
 (segment (start 119.9 53.8) (end 119.9 54.294974) (width 0.25) (layer F.Cu) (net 24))
 (segment (start 118.444974 55.75) (end 112 55.75) (width 0.25) (layer F.Cu) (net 24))
 (segment (start 109.283561 58.466439) (end 112 55.75) (width 0.25) (layer F.Cu) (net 24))
 (segment (start 109.283561 66.203849) (end 109.283561 58.466439) (width 0.25) (layer F.Cu) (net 24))
 (segment (start 108.458062 67.029348) (end 109.283561 66.203849) (width 0.25) (layer F.Cu) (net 24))
 (segment (start 104.193935 71.293475) (end 108.458062 67.029348) (width 0.25) (layer F.Cu) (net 24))
 (segment (start 104.193935 73.979649) (end 104.193935 71.293475) (width 0.25) (layer F.Cu) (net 24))
 (segment (start 125.7 51) (end 130.449989 55.749989) (width 0.25) (layer F.Cu) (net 24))
 (segment (start 130.449989 55.749989) (end 158.899989 55.749989) (width 0.25) (layer F.Cu) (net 24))
 (segment (start 164.312741 61.162741) (end 174.998042 61.162741) (width 0.25) (layer F.Cu) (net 24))
 (segment (start 158.899989 55.749989) (end 164.312741 61.162741) (width 0.25) (layer F.Cu) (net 24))
 (segment (start 120.75 53.650998) (end 120.75 53.8) (width 0.25) (layer F.Cu) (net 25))
 (segment (start 119.9 52.800998) (end 120.75 53.650998) (width 0.25) (layer F.Cu) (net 25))
 (segment (start 119.9 52.45) (end 119.9 52.800998) (width 0.25) (layer F.Cu) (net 25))
 (segment (start 111 71.3) (end 111 57.7) (width 0.25) (layer F.Cu) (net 25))
 (segment (start 109.7 72.6) (end 111 71.3) (width 0.25) (layer F.Cu) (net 25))
 (segment (start 120.75 54.294974) (end 120.75 53.8) (width 0.25) (layer F.Cu) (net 25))
 (segment (start 118.844965 56.200009) (end 120.75 54.294974) (width 0.25) (layer F.Cu) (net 25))
 (segment (start 111 57.7) (end 112.499991 56.200009) (width 0.25) (layer F.Cu) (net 25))
 (segment (start 112.499991 56.200009) (end 118.844965 56.200009) (width 0.25) (layer F.Cu) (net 25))
 (segment (start 160.759315 133.375) (end 160.409325 133.72499) (width 0.25) (layer F.Cu) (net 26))
 (segment (start 161.325 133.375) (end 160.759315 133.375) (width 0.25) (layer F.Cu) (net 26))
 (segment (start 160.409325 133.72499) (end 110.84999 133.72499) (width 0.25) (layer F.Cu) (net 26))
 (segment (start 110.84999 133.72499) (end 110.575 133.45) (width 0.25) (layer F.Cu) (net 26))
 (segment (start 164.354701 136.310078) (end 184.410078 136.310078) (width 0.25) (layer F.Cu) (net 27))
 (segment (start 184.410078 136.310078) (end 184.825 136.725) (width 0.25) (layer F.Cu) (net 27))
 (segment (start 192.9331 134.025) (end 197.623022 129.335078) (width 0.25) (layer F.Cu) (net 27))
 (segment (start 185.925 134.025) (end 192.9331 134.025) (width 0.25) (layer F.Cu) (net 27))
 (segment (start 190.123022 135.585078) (end 163.985078 135.585078) (width 0.25) (layer F.Cu) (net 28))
 (segment (start 163.985078 135.585078) (end 163.8 135.4) (width 0.25) (layer F.Cu) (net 28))
 (segment (start 118.2 52.45) (end 118.2 53.8) (width 0.25) (layer F.Cu) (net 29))
 (segment (start 122.45 52.45) (end 122.45 53.8) (width 0.25) (layer F.Cu) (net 29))
 (segment (start 122.45 51.955026) (end 122.45 52.45) (width 0.25) (layer F.Cu) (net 29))
 (segment (start 122.269973 51.774999) (end 122.45 51.955026) (width 0.25) (layer F.Cu) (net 29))
 (segment (start 118.380027 51.774999) (end 122.269973 51.774999) (width 0.25) (layer F.Cu) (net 29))
 (segment (start 118.2 51.955026) (end 118.380027 51.774999) (width 0.25) (layer F.Cu) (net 29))
 (segment (start 118.2 52.45) (end 118.2 51.955026) (width 0.25) (layer F.Cu) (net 29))
 (segment (start 136.354999 58.195001) (end 135.35 59.2) (width 0.25) (layer F.Cu) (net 29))
 (segment (start 124.700997 56.199999) (end 135.248001 56.199999) (width 0.25) (layer F.Cu) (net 29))
 (segment (start 122.624999 54.124001) (end 124.700997 56.199999) (width 0.25) (layer F.Cu) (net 29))
 (segment (start 122.624999 53.949999) (end 122.624999 54.124001) (width 0.25) (layer F.Cu) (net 29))
 (segment (start 135.248001 56.199999) (end 136.354999 57.306997) (width 0.25) (layer F.Cu) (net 29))
 (segment (start 122.475 53.8) (end 122.624999 53.949999) (width 0.25) (layer F.Cu) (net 29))
 (segment (start 136.354999 57.306997) (end 136.354999 58.195001) (width 0.25) (layer F.Cu) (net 29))
 (segment (start 122.45 53.8) (end 122.475 53.8) (width 0.25) (layer F.Cu) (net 29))
 (segment (start 192.3 114.799695) (end 192.3 115.18859) (width 0.25) (layer F.Cu) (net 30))
 (segment (start 192.43695 114.662745) (end 192.3 114.799695) (width 0.25) (layer F.Cu) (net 30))
 (segment (start 192.3 115.18859) (end 183.569295 123.919295) (width 0.25) (layer F.Cu) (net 30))
 (segment (start 183.569295 123.919295) (end 176.248603 131.239987) (width 0.25) (layer F.Cu) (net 30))
 (segment (start 158.946475 131.239988) (end 158.261513 131.92495) (width 0.25) (layer F.Cu) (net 30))
 (segment (start 176.248603 131.239987) (end 158.946475 131.239988) (width 0.25) (layer F.Cu) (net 30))
 (segment (start 158.261513 131.92495) (end 131.89675 131.92495) (width 0.25) (layer F.Cu) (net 30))
 (segment (start 131.89675 131.92495) (end 131.369053 131.397253) (width 0.25) (layer F.Cu) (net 30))
 (segment (start 188.663618 52.424972) (end 186.75 52.424972) (width 0.25) (layer F.Cu) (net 30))
 (segment (start 189.563591 51.524999) (end 188.663618 52.424972) (width 0.25) (layer F.Cu) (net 30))
 (segment (start 196.2 53) (end 194.724999 51.524999) (width 0.25) (layer F.Cu) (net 30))
 (segment (start 194.724999 51.524999) (end 189.563591 51.524999) (width 0.25) (layer F.Cu) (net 30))
 (segment (start 186.75 52.45) (end 186.500038 52.699962) (width 0.25) (layer F.Cu) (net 30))
 (segment (start 186.75 52.424972) (end 186.75 52.45) (width 0.25) (layer F.Cu) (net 30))
 (segment (start 165.740675 52.699962) (end 186.500038 52.699962) (width 0.25) (layer F.Cu) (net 30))
 (segment (start 165.465685 52.424972) (end 165.740675 52.699962) (width 0.25) (layer F.Cu) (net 30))
 (segment (start 164.9 52.424972) (end 165.465685 52.424972) (width 0.25) (layer F.Cu) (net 30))
 (segment (start 134.9 95.48) (end 132.25002 98.12998) (width 0.25) (layer F.Cu) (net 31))
 (segment (start 132.25002 98.12998) (end 132.25002 99.8) (width 0.25) (layer F.Cu) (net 31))
 (segment (start 132.25002 125.825) (end 133.800019 127.374999) (width 0.25) (layer F.Cu) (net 31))
 (segment (start 178.840771 126.986103) (end 190.347437 115.479437) (width 0.25) (layer F.Cu) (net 31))
 (segment (start 178.451875 127.374999) (end 178.840771 126.986103) (width 0.25) (layer F.Cu) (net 31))
 (segment (start 133.800019 127.374999) (end 178.451875 127.374999) (width 0.25) (layer F.Cu) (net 31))
 (segment (start 131.75 92.33) (end 134.9 95.48) (width 0.25) (layer F.Cu) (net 31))
 (segment (start 131.75 90.3) (end 131.75 92.33) (width 0.25) (layer F.Cu) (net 31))
 (segment (start 114.643216 60.611846) (end 115.580062 59.675) (width 0.25) (layer F.Cu) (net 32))
 (segment (start 113.511846 60.611846) (end 114.643216 60.611846) (width 0.25) (layer F.Cu) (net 32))
 (segment (start 132.15 59.675) (end 115.580062 59.675) (width 0.25) (layer F.Cu) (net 32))
 (segment (start 134.9 56.925) (end 132.15 59.675) (width 0.25) (layer F.Cu) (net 32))
 (segment (start 131.80001 130.211146) (end 133.063804 131.47494) (width 0.25) (layer F.Cu) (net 32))
 (segment (start 133.063804 131.47494) (end 148.575 131.47494) (width 0.25) (layer F.Cu) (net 32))
 (segment (start 158.075113 131.47494) (end 158.760076 130.789979) (width 0.25) (layer F.Cu) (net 32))
 (segment (start 148.575 131.47494) (end 158.075113 131.47494) (width 0.25) (layer F.Cu) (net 32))
 (segment (start 158.760076 130.789979) (end 176.062201 130.789979) (width 0.25) (layer F.Cu) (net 32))
 (segment (start 176.062201 130.789979) (end 191.372749 115.479431) (width 0.25) (layer F.Cu) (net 32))
 (segment (start 191.372749 115.479431) (end 191.372749 115.090535) (width 0.25) (layer F.Cu) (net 32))
 (segment (start 131.29999 90.94999) (end 123.75 83.4) (width 0.25) (layer F.Cu) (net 32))
 (segment (start 131.80001 94.35) (end 131.29999 93.84998) (width 0.25) (layer F.Cu) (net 32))
 (segment (start 131.29999 93.84998) (end 131.29999 90.94999) (width 0.25) (layer F.Cu) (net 32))
 (segment (start 113.511846 61.743216) (end 113.511846 60.611846) (width 0.25) (layer F.Cu) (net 32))
 (segment (start 113.511846 62.276848) (end 113.511846 61.743216) (width 0.25) (layer F.Cu) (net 32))
 (segment (start 121.034999 69.800001) (end 113.511846 62.276848) (width 0.25) (layer F.Cu) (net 32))
 (segment (start 122.800001 69.800001) (end 121.034999 69.800001) (width 0.25) (layer F.Cu) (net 32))
 (segment (start 123.2 70.2) (end 122.800001 69.800001) (width 0.25) (layer F.Cu) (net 32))
 (segment (start 136.9 78.67501) (end 162.82499 78.67501) (width 0.25) (layer F.Cu) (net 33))
 (segment (start 162.82499 78.67501) (end 163.025 78.475) (width 0.25) (layer F.Cu) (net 33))
 (segment (start 162.824999 94.4) (end 163.349999 93.875) (width 0.25) (layer F.Cu) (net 33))
 (segment (start 163.349999 93.875) (end 190.47493 93.875) (width 0.25) (layer F.Cu) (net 33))
 (segment (start 190.863437 81.838437) (end 190.863437 75.228743) (width 0.25) (layer F.Cu) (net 33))
 (segment (start 190.863437 75.228743) (end 190.567347 74.932653) (width 0.25) (layer F.Cu) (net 33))
 (segment (start 189.682018 70.482018) (end 187.6 68.4) (width 0.25) (layer F.Cu) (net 33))
 (segment (start 189.682018 71.690668) (end 189.682018 70.482018) (width 0.25) (layer F.Cu) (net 33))
 (segment (start 131.190685 132.09997) (end 131.465675 132.37496) (width 0.25) (layer F.Cu) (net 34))
 (segment (start 130.625 132.09997) (end 131.190685 132.09997) (width 0.25) (layer F.Cu) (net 34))
 (segment (start 131.465675 132.37496) (end 138.6 132.37496) (width 0.25) (layer F.Cu) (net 34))
 (segment (start 138.6 132.37496) (end 154.22504 132.37496) (width 0.25) (layer F.Cu) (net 34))
 (segment (start 154.22504 132.37496) (end 158.447913 132.37496) (width 0.25) (layer F.Cu) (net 34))
 (segment (start 158.447913 132.37496) (end 159.132876 131.689997) (width 0.25) (layer F.Cu) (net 34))
 (segment (start 159.132876 131.689997) (end 172.384697 131.689997) (width 0.25) (layer F.Cu) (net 34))
 (segment (start 172.384697 131.689997) (end 176.435003 131.689997) (width 0.25) (layer F.Cu) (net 34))
 (segment (start 176.435003 131.689997) (end 193.525 114.6) (width 0.25) (layer F.Cu) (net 34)))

